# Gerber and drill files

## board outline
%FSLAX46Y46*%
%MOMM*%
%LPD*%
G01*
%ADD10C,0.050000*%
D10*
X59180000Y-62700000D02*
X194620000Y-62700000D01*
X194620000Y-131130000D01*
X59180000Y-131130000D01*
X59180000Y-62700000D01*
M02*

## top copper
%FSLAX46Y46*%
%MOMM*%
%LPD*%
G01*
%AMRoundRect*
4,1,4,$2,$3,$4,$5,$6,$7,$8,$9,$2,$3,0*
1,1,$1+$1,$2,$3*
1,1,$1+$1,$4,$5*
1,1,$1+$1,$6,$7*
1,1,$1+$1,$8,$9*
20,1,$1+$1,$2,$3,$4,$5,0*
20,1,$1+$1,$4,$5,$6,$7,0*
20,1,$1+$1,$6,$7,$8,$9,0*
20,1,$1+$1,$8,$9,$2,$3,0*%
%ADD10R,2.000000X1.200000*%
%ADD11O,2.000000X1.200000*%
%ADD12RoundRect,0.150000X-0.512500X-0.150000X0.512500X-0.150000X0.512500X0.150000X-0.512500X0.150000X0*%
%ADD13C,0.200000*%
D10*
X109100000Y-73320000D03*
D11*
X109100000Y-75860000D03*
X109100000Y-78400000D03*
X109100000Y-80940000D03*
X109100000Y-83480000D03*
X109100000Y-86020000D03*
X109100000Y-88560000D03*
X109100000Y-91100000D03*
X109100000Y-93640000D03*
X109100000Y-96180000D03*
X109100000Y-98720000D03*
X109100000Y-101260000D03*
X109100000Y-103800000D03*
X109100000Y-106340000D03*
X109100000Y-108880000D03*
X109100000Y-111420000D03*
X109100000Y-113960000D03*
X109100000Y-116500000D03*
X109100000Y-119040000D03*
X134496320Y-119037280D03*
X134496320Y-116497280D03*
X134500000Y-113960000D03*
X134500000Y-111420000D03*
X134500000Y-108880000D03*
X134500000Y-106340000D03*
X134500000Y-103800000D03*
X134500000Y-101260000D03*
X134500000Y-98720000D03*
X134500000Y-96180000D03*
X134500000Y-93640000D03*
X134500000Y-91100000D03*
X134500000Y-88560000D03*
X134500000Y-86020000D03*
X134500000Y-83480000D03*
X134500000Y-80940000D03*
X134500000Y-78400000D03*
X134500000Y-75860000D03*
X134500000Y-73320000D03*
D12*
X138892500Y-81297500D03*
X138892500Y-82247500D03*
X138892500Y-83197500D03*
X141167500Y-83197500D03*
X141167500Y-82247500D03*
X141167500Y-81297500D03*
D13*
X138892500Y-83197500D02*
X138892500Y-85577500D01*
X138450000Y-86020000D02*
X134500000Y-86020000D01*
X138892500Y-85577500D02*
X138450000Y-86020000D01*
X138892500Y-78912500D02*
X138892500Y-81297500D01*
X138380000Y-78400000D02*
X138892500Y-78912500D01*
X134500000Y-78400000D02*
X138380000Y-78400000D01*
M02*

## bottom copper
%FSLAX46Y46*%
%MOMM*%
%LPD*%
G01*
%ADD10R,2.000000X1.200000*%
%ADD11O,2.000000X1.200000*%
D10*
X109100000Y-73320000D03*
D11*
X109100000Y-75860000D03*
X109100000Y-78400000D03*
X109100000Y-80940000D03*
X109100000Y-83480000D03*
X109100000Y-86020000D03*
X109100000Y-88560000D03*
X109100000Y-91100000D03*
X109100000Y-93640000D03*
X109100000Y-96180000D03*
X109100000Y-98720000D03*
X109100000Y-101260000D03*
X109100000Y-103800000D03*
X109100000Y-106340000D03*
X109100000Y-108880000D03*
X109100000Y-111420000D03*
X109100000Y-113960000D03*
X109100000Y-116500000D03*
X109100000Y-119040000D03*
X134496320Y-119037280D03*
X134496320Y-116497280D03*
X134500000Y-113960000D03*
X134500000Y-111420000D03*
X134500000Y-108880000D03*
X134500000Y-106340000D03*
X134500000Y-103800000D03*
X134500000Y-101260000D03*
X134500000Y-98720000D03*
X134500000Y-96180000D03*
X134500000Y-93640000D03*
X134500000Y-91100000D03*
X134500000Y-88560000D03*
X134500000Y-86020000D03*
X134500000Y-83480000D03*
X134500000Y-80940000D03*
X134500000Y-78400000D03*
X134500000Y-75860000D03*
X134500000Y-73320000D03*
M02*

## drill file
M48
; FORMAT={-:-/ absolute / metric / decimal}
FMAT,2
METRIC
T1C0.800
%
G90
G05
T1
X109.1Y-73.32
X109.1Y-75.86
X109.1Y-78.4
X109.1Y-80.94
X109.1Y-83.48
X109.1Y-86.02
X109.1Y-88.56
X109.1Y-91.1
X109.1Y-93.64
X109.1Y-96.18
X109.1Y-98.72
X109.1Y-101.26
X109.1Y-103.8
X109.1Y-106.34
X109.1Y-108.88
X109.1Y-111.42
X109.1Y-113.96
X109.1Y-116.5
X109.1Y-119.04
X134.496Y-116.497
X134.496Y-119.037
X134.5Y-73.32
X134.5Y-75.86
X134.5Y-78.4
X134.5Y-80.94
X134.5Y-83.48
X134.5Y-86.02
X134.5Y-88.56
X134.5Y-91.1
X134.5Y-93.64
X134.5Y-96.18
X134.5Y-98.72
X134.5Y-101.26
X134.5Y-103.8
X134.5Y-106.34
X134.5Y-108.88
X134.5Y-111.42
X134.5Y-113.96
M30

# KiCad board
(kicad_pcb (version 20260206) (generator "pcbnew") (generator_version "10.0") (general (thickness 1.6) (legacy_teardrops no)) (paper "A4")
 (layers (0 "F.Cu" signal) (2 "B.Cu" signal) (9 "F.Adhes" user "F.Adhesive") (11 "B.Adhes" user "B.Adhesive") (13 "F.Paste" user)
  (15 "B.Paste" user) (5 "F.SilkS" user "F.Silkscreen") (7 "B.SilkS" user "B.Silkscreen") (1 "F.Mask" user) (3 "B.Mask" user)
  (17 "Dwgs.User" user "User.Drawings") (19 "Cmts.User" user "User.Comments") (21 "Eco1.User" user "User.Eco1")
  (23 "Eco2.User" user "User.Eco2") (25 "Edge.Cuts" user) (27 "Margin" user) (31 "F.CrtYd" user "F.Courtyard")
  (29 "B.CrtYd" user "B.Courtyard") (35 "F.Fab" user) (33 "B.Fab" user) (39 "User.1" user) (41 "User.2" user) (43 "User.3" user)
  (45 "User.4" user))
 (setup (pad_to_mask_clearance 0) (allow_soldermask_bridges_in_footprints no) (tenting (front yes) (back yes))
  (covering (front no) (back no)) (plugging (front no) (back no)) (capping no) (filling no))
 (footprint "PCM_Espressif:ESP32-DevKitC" (layer "F.Cu") (at 109.1 73.32)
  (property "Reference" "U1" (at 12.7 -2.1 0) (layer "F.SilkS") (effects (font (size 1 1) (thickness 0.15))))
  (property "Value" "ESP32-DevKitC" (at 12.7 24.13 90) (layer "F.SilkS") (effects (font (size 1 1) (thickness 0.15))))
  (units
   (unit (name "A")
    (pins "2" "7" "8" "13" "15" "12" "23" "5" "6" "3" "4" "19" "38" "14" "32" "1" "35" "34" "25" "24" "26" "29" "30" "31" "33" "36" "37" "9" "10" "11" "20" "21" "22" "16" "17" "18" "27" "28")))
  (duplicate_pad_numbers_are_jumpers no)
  (pad "1" thru_hole rect (at 0 0 270) (size 1.2 2) (drill 0.8) (layers "*.Cu" "*.Mask") (remove_unused_layers no) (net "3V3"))
  (pad "2" thru_hole oval (at 0 2.54 270) (size 1.2 2) (drill 0.8) (layers "*.Cu" "*.Mask") (remove_unused_layers no)
   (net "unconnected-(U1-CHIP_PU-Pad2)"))
  (pad "3" thru_hole oval (at 0 5.08 270) (size 1.2 2) (drill 0.8) (layers "*.Cu" "*.Mask") (remove_unused_layers no)
   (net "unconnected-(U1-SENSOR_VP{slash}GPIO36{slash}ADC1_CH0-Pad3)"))
  (pad "4" thru_hole oval (at 0 7.62 270) (size 1.2 2) (drill 0.8) (layers "*.Cu" "*.Mask") (remove_unused_layers no)
   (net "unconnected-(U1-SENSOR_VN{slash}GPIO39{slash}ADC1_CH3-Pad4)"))
  (pad "5" thru_hole oval (at 0 10.16 270) (size 1.2 2) (drill 0.8) (layers "*.Cu" "*.Mask") (remove_unused_layers no)
   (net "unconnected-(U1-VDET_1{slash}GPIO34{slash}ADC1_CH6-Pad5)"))
  (pad "6" thru_hole oval (at 0 12.7 270) (size 1.2 2) (drill 0.8) (layers "*.Cu" "*.Mask") (remove_unused_layers no)
   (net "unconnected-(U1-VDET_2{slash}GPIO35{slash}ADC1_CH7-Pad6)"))
  (pad "7" thru_hole oval (at 0 15.24 270) (size 1.2 2) (drill 0.8) (layers "*.Cu" "*.Mask") (remove_unused_layers no)
   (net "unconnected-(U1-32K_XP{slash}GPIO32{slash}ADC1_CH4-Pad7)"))
  (pad "8" thru_hole oval (at 0 17.78 270) (size 1.2 2) (drill 0.8) (layers "*.Cu" "*.Mask") (remove_unused_layers no)
   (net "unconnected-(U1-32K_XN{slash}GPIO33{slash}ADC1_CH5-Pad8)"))
  (pad "9" thru_hole oval (at 0 20.32 270) (size 1.2 2) (drill 0.8) (layers "*.Cu" "*.Mask") (remove_unused_layers no) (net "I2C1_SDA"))
  (pad "10" thru_hole oval (at 0 22.86 270) (size 1.2 2) (drill 0.8) (layers "*.Cu" "*.Mask") (remove_unused_layers no) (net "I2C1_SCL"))
  (pad "11" thru_hole oval (at 0 25.4 270) (size 1.2 2) (drill 0.8) (layers "*.Cu" "*.Mask") (remove_unused_layers no)
   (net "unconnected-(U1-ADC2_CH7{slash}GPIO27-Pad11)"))
  (pad "12" thru_hole oval (at 0 27.94 270) (size 1.2 2) (drill 0.8) (layers "*.Cu" "*.Mask") (remove_unused_layers no)
   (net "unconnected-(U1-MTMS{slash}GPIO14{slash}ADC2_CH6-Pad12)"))
  (pad "13" thru_hole oval (at 0 30.48 270) (size 1.2 2) (drill 0.8) (layers "*.Cu" "*.Mask") (remove_unused_layers no)
   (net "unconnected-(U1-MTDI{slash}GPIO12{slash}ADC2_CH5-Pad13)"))
  (pad "14" thru_hole oval (at 0 33.02 270) (size 1.2 2) (drill 0.8) (layers "*.Cu" "*.Mask") (remove_unused_layers no) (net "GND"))
  (pad "15" thru_hole oval (at 0 35.56 270) (size 1.2 2) (drill 0.8) (layers "*.Cu" "*.Mask") (remove_unused_layers no)
   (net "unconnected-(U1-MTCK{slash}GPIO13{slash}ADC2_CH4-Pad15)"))
  (pad "16" thru_hole oval (at 0 38.1 270) (size 1.2 2) (drill 0.8) (layers "*.Cu" "*.Mask") (remove_unused_layers no)
   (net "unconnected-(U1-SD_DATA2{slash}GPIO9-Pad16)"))
  (pad "17" thru_hole oval (at 0 40.64 270) (size 1.2 2) (drill 0.8) (layers "*.Cu" "*.Mask") (remove_unused_layers no)
   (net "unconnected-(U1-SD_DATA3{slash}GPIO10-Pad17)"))
  (pad "18" thru_hole oval (at 0 43.18 270) (size 1.2 2) (drill 0.8) (layers "*.Cu" "*.Mask") (remove_unused_layers no)
   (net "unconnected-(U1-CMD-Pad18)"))
  (pad "19" thru_hole oval (at 0 45.72 270) (size 1.2 2) (drill 0.8) (layers "*.Cu" "*.Mask") (remove_unused_layers no)
   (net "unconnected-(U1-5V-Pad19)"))
  (pad "20" thru_hole oval (at 25.39632 45.71728 270) (size 1.2 2) (drill 0.8) (layers "*.Cu" "*.Mask") (remove_unused_layers no)
   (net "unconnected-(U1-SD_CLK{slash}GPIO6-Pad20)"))
  (pad "21" thru_hole oval (at 25.39632 43.17728 270) (size 1.2 2) (drill 0.8) (layers "*.Cu" "*.Mask") (remove_unused_layers no)
   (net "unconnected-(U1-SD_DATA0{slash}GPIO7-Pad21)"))
  (pad "22" thru_hole oval (at 25.4 40.64 270) (size 1.2 2) (drill 0.8) (layers "*.Cu" "*.Mask") (remove_unused_layers no)
   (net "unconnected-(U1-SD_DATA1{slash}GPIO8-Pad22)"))
  (pad "23" thru_hole oval (at 25.4 38.1 270) (size 1.2 2) (drill 0.8) (layers "*.Cu" "*.Mask") (remove_unused_layers no)
   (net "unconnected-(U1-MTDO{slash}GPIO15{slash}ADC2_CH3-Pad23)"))
  (pad "24" thru_hole oval (at 25.4 35.56 270) (size 1.2 2) (drill 0.8) (layers "*.Cu" "*.Mask") (remove_unused_layers no)
   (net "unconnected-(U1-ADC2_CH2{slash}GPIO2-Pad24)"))
  (pad "25" thru_hole oval (at 25.4 33.02 270) (size 1.2 2) (drill 0.8) (layers "*.Cu" "*.Mask") (remove_unused_layers no)
   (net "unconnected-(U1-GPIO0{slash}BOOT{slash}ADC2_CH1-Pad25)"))
  (pad "26" thru_hole oval (at 25.4 30.48 270) (size 1.2 2) (drill 0.8) (layers "*.Cu" "*.Mask") (remove_unused_layers no)
   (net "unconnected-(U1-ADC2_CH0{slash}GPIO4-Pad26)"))
  (pad "27" thru_hole oval (at 25.4 27.94 270) (size 1.2 2) (drill 0.8) (layers "*.Cu" "*.Mask") (remove_unused_layers no)
   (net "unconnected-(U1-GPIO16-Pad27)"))
  (pad "28" thru_hole oval (at 25.4 25.4 270) (size 1.2 2) (drill 0.8) (layers "*.Cu" "*.Mask") (remove_unused_layers no)
   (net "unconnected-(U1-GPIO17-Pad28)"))
  (pad "29" thru_hole oval (at 25.4 22.86 270) (size 1.2 2) (drill 0.8) (layers "*.Cu" "*.Mask") (remove_unused_layers no)
   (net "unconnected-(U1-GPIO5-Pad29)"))
  (pad "30" thru_hole oval (at 25.4 20.32 270) (size 1.2 2) (drill 0.8) (layers "*.Cu" "*.Mask") (remove_unused_layers no)
   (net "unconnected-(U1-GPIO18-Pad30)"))
  (pad "31" thru_hole oval (at 25.4 17.78 270) (size 1.2 2) (drill 0.8) (layers "*.Cu" "*.Mask") (remove_unused_layers no)
   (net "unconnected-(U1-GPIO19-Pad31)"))
  (pad "32" thru_hole oval (at 25.4 15.24 270) (size 1.2 2) (drill 0.8) (layers "*.Cu" "*.Mask") (remove_unused_layers no) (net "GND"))
  (pad "33" thru_hole oval (at 25.4 12.7 270) (size 1.2 2) (drill 0.8) (layers "*.Cu" "*.Mask") (remove_unused_layers no) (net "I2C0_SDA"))
  (pad "34" thru_hole oval (at 25.4 10.16 270) (size 1.2 2) (drill 0.8) (layers "*.Cu" "*.Mask") (remove_unused_layers no)
   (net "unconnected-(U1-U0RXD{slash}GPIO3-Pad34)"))
  (pad "35" thru_hole oval (at 25.4 7.62 270) (size 1.2 2) (drill 0.8) (layers "*.Cu" "*.Mask") (remove_unused_layers no)
   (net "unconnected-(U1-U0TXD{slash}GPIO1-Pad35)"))
  (pad "36" thru_hole oval (at 25.4 5.08 270) (size 1.2 2) (drill 0.8) (layers "*.Cu" "*.Mask") (remove_unused_layers no) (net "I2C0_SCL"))
  (pad "37" thru_hole oval (at 25.4 2.54 270) (size 1.2 2) (drill 0.8) (layers "*.Cu" "*.Mask") (remove_unused_layers no)
   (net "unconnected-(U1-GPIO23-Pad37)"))
  (pad "38" thru_hole oval (at 25.4 0 270) (size 1.2 2) (drill 0.8) (layers "*.Cu" "*.Mask") (remove_unused_layers no) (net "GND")))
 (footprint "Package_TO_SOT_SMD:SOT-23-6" (layer "F.Cu") (at 140.03 82.2475)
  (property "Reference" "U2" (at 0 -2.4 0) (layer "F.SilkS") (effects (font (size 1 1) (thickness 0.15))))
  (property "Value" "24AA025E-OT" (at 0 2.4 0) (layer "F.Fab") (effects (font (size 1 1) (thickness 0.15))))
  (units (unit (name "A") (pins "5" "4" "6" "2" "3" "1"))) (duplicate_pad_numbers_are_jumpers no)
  (pad "1" smd roundrect (at -1.1375 -0.95) (size 1.325 0.6) (layers "F.Cu" "F.Mask" "F.Paste") (roundrect_rratio 0.25) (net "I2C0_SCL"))
  (pad "2" smd roundrect (at -1.1375 0) (size 1.325 0.6) (layers "F.Cu" "F.Mask" "F.Paste") (roundrect_rratio 0.25) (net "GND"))
  (pad "3" smd roundrect (at -1.1375 0.95) (size 1.325 0.6) (layers "F.Cu" "F.Mask" "F.Paste") (roundrect_rratio 0.25) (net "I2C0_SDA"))
  (pad "4" smd roundrect (at 1.1375 0.95) (size 1.325 0.6) (layers "F.Cu" "F.Mask" "F.Paste") (roundrect_rratio 0.25) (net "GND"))
  (pad "5" smd roundrect (at 1.1375 0) (size 1.325 0.6) (layers "F.Cu" "F.Mask" "F.Paste") (roundrect_rratio 0.25) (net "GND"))
  (pad "6" smd roundrect (at 1.1375 -0.95) (size 1.325 0.6) (layers "F.Cu" "F.Mask" "F.Paste") (roundrect_rratio 0.25) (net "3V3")))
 (gr_rect (start 59.18 62.7) (end 194.62 131.13) (stroke (width 0.05) (type default)) (fill no) (layer "Edge.Cuts"))
 (segment (start 138.8925 83.1975) (end 138.8925 85.5775) (width 0.2) (layer "F.Cu") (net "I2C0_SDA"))
 (segment (start 138.45 86.02) (end 134.5 86.02) (width 0.2) (layer "F.Cu") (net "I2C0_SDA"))
 (segment (start 138.8925 85.5775) (end 138.45 86.02) (width 0.2) (layer "F.Cu") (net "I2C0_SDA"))
 (segment (start 138.8925 78.9125) (end 138.8925 81.2975) (width 0.2) (layer "F.Cu") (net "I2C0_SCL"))
 (segment (start 138.38 78.4) (end 138.8925 78.9125) (width 0.2) (layer "F.Cu") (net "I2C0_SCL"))
 (segment (start 134.5 78.4) (end 138.38 78.4) (width 0.2) (layer "F.Cu") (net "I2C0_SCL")))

